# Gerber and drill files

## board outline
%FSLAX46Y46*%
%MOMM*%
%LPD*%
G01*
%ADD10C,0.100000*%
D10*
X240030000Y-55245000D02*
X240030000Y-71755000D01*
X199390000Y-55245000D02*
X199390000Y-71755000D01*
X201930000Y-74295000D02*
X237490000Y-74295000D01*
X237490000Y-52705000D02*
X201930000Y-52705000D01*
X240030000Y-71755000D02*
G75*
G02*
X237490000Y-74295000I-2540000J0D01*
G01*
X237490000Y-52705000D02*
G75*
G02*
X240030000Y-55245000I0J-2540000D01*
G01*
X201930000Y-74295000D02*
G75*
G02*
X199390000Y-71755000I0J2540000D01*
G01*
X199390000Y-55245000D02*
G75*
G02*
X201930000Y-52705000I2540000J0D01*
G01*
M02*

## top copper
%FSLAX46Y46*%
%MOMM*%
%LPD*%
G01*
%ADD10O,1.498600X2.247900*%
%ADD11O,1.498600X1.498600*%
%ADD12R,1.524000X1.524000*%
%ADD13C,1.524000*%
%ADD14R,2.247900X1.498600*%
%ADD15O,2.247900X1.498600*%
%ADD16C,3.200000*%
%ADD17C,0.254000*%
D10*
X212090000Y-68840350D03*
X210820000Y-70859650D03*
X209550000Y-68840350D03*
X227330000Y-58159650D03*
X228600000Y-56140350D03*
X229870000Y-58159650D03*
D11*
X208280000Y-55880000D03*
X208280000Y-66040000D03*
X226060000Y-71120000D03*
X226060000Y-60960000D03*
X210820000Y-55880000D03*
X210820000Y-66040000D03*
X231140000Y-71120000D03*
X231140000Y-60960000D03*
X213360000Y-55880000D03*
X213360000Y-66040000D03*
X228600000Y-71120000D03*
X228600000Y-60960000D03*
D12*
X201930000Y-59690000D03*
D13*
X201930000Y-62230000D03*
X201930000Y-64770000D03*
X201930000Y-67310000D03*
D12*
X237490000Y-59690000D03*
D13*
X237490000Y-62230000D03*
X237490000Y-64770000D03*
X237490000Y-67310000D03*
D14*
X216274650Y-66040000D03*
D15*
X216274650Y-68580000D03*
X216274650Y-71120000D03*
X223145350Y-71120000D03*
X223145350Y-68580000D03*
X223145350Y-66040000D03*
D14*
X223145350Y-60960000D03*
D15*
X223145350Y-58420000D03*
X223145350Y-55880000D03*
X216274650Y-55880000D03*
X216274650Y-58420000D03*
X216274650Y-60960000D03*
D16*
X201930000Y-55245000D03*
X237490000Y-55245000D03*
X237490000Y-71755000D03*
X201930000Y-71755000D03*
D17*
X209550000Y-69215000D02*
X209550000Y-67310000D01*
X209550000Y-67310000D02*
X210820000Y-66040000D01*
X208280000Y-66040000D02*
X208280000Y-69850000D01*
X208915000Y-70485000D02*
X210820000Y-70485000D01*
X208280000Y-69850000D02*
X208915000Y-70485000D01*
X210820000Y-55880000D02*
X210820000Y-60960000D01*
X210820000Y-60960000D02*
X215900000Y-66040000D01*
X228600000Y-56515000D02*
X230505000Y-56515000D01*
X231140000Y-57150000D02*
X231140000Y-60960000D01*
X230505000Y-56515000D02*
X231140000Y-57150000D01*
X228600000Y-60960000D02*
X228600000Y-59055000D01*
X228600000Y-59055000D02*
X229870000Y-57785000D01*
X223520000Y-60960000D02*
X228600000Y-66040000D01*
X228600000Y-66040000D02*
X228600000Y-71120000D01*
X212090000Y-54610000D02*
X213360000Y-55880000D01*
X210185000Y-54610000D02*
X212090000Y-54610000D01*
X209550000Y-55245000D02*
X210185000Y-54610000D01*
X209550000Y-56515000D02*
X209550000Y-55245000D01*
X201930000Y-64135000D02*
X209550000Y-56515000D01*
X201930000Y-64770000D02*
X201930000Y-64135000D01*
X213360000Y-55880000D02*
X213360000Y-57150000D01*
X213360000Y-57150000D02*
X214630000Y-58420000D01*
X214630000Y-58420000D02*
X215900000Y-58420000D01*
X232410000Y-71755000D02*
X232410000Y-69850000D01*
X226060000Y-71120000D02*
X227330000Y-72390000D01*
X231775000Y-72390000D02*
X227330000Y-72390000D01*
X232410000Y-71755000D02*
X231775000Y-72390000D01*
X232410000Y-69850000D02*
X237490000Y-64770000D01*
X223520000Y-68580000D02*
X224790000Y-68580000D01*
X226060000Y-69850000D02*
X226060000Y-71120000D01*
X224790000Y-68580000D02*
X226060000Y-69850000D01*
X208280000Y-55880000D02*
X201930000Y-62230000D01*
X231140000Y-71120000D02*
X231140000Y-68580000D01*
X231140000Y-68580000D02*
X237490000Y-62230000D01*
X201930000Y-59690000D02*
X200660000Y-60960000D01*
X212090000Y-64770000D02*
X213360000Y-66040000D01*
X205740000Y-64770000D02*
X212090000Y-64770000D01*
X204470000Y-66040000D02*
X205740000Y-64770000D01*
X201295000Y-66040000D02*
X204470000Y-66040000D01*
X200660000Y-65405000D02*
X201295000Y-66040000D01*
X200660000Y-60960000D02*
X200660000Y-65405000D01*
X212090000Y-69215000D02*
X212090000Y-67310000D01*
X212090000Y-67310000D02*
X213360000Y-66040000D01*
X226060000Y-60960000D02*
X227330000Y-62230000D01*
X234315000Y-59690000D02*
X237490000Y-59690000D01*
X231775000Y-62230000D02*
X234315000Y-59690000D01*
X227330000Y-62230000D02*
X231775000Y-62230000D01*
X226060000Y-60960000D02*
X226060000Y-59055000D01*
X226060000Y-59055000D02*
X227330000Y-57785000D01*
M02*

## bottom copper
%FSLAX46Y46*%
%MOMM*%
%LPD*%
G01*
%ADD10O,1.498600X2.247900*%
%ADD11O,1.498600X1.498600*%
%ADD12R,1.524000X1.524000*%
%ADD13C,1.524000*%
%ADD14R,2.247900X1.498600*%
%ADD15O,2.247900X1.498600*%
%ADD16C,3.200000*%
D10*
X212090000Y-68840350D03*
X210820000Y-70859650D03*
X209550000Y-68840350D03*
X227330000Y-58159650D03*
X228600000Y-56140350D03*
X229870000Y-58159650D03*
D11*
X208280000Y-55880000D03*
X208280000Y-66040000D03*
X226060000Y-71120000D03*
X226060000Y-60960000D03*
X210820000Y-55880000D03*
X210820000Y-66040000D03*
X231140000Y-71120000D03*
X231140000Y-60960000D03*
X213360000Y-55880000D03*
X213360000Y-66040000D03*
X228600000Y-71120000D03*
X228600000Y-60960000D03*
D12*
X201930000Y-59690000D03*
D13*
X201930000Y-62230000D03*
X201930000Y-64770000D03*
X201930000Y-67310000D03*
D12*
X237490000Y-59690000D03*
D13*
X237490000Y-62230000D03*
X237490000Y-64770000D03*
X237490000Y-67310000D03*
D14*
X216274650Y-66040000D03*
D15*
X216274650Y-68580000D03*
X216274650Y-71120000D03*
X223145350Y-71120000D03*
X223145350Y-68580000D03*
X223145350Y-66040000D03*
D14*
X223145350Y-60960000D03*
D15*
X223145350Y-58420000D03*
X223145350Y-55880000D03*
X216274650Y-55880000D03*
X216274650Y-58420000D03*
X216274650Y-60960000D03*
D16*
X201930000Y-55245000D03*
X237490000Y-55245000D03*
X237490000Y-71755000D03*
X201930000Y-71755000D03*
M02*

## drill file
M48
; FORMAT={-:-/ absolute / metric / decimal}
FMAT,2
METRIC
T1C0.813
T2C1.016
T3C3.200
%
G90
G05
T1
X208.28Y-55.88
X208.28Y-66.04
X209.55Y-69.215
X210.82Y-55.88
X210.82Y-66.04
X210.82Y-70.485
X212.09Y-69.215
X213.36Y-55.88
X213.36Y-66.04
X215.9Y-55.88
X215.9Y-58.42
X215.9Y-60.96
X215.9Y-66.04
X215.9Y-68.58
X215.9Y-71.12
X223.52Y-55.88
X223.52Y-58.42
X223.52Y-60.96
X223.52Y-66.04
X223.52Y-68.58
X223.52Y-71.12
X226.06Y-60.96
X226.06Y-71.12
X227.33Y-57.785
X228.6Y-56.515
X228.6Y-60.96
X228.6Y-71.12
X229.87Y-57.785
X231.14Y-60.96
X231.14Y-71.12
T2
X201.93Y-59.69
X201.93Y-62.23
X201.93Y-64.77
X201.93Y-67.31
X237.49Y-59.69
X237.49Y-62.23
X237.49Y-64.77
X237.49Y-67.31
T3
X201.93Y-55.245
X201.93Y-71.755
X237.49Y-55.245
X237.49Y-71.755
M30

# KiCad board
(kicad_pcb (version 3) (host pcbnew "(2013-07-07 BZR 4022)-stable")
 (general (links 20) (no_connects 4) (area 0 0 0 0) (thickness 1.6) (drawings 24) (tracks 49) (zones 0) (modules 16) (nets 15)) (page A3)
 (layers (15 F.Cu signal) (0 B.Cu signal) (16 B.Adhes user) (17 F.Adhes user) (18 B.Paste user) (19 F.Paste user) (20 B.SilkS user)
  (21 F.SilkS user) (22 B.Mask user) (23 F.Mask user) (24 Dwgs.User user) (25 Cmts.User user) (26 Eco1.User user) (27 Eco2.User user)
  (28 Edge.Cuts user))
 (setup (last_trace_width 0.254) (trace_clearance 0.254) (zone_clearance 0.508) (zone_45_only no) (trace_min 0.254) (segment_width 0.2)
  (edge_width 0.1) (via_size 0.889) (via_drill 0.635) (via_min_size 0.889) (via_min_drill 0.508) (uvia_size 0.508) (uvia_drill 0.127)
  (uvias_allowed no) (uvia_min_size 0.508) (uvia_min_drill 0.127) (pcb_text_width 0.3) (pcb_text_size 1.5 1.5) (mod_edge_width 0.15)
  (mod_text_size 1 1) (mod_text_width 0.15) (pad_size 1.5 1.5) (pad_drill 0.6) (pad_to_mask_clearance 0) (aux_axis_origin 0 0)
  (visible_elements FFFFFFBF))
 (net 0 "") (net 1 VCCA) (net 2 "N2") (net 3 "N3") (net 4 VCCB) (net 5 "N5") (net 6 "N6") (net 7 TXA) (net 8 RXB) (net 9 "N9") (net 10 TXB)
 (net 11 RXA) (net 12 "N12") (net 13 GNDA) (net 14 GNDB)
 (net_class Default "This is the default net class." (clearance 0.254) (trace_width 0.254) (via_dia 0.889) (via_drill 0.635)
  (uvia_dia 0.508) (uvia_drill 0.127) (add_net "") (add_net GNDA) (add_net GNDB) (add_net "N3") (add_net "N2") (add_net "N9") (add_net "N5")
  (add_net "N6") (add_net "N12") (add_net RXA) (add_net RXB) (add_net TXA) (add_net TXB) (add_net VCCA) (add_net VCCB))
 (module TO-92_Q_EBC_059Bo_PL (layer F.Cu) (at 212.09 69.215)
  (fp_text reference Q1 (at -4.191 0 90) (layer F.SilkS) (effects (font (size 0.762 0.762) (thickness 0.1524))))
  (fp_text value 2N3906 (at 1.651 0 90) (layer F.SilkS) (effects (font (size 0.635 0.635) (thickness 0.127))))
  (pad 1 thru_hole oval (at 0 0) (size 1.4986 2.2479) (drill 0.8128 (offset 0 -0.37465)) (layers *.Cu *.Mask F.SilkS) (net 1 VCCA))
  (pad 2 thru_hole oval (at -1.27 1.27) (size 1.4986 2.2479) (drill 0.8128 (offset 0 0.37465)) (layers *.Cu *.Mask F.SilkS) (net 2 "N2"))
  (pad 3 thru_hole oval (at -2.54 0) (size 1.4986 2.2479) (drill 0.8128 (offset 0 -0.37465)) (layers *.Cu *.Mask F.SilkS) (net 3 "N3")))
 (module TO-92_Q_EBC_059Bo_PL (layer F.Cu) (at 227.33 57.785 180)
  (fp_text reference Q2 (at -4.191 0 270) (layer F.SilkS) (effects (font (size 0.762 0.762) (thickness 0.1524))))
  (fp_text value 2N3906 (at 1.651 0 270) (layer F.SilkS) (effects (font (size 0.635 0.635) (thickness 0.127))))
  (pad 1 thru_hole oval (at 0 0 180) (size 1.4986 2.2479) (drill 0.8128 (offset 0 -0.37465)) (layers *.Cu *.Mask F.SilkS) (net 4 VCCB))
  (pad 2 thru_hole oval (at -1.27 1.27 180) (size 1.4986 2.2479) (drill 0.8128 (offset 0 0.37465)) (layers *.Cu *.Mask F.SilkS) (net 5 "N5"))
  (pad 3 thru_hole oval (at -2.54 0 180) (size 1.4986 2.2479) (drill 0.8128 (offset 0 -0.37465)) (layers *.Cu *.Mask F.SilkS) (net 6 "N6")))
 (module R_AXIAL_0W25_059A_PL (layer F.Cu) (at 208.28 55.88 270) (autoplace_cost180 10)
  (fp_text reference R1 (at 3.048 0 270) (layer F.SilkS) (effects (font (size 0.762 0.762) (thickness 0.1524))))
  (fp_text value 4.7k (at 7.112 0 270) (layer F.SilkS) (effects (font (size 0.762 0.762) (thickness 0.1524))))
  (pad 1 thru_hole oval (at 0 0 270) (size 1.4986 1.4986) (drill 0.8128) (layers *.Cu *.Mask F.SilkS) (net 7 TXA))
  (pad 2 thru_hole oval (at 10.16 0 270) (size 1.4986 1.4986) (drill 0.8128) (layers *.Cu *.Mask F.SilkS) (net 2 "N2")))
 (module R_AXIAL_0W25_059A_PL (layer F.Cu) (at 226.06 71.12 90) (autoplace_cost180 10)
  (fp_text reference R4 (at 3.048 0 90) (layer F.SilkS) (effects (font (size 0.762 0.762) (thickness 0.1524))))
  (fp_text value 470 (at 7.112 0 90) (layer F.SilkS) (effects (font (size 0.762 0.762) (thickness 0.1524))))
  (pad 1 thru_hole oval (at 0 0 90) (size 1.4986 1.4986) (drill 0.8128) (layers *.Cu *.Mask F.SilkS) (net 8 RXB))
  (pad 2 thru_hole oval (at 10.16 0 90) (size 1.4986 1.4986) (drill 0.8128) (layers *.Cu *.Mask F.SilkS) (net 4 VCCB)))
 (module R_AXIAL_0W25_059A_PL (layer F.Cu) (at 210.82 55.88 270) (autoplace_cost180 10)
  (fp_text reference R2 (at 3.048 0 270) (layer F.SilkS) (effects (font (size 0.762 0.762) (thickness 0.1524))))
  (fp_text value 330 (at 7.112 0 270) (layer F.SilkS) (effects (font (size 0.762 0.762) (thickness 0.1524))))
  (pad 1 thru_hole oval (at 0 0 270) (size 1.4986 1.4986) (drill 0.8128) (layers *.Cu *.Mask F.SilkS) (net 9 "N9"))
  (pad 2 thru_hole oval (at 10.16 0 270) (size 1.4986 1.4986) (drill 0.8128) (layers *.Cu *.Mask F.SilkS) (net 3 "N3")))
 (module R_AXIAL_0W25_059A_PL (layer F.Cu) (at 231.14 71.12 90) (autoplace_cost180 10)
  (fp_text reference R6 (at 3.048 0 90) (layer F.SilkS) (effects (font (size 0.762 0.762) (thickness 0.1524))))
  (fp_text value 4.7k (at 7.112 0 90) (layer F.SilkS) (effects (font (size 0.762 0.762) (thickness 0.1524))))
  (pad 1 thru_hole oval (at 0 0 90) (size 1.4986 1.4986) (drill 0.8128) (layers *.Cu *.Mask F.SilkS) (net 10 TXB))
  (pad 2 thru_hole oval (at 10.16 0 90) (size 1.4986 1.4986) (drill 0.8128) (layers *.Cu *.Mask F.SilkS) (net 5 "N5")))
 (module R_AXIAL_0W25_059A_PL (layer F.Cu) (at 213.36 55.88 270) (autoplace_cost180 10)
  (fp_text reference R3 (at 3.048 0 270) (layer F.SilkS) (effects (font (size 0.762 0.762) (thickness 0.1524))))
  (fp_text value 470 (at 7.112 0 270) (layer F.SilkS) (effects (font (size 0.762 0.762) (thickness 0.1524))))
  (pad 1 thru_hole oval (at 0 0 270) (size 1.4986 1.4986) (drill 0.8128) (layers *.Cu *.Mask F.SilkS) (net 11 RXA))
  (pad 2 thru_hole oval (at 10.16 0 270) (size 1.4986 1.4986) (drill 0.8128) (layers *.Cu *.Mask F.SilkS) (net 1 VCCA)))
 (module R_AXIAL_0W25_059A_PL (layer F.Cu) (at 228.6 71.12 90) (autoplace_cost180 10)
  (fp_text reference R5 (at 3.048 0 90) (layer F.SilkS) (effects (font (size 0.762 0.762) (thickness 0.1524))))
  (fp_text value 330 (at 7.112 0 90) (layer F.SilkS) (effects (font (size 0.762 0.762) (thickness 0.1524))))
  (pad 1 thru_hole oval (at 0 0 90) (size 1.4986 1.4986) (drill 0.8128) (layers *.Cu *.Mask F.SilkS) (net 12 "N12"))
  (pad 2 thru_hole oval (at 10.16 0 90) (size 1.4986 1.4986) (drill 0.8128) (layers *.Cu *.Mask F.SilkS) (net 6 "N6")))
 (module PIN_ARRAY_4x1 (layer F.Cu) (at 201.93 63.5 270)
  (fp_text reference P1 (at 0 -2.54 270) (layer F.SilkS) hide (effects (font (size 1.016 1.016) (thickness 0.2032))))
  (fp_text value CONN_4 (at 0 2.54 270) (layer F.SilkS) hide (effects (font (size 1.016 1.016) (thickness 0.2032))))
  (pad 1 thru_hole rect (at -3.81 0 270) (size 1.524 1.524) (drill 1.016) (layers *.Cu *.Mask F.SilkS) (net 1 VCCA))
  (pad 2 thru_hole circle (at -1.27 0 270) (size 1.524 1.524) (drill 1.016) (layers *.Cu *.Mask F.SilkS) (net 7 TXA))
  (pad 3 thru_hole circle (at 1.27 0 270) (size 1.524 1.524) (drill 1.016) (layers *.Cu *.Mask F.SilkS) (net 11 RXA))
  (pad 4 thru_hole circle (at 3.81 0 270) (size 1.524 1.524) (drill 1.016) (layers *.Cu *.Mask F.SilkS) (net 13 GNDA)))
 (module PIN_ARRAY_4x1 (layer F.Cu) (at 237.49 63.5 270)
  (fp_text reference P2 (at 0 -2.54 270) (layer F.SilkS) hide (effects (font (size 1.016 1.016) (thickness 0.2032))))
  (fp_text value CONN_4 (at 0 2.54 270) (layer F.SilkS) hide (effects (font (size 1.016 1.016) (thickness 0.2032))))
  (pad 1 thru_hole rect (at -3.81 0 270) (size 1.524 1.524) (drill 1.016) (layers *.Cu *.Mask F.SilkS) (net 4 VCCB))
  (pad 2 thru_hole circle (at -1.27 0 270) (size 1.524 1.524) (drill 1.016) (layers *.Cu *.Mask F.SilkS) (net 10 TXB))
  (pad 3 thru_hole circle (at 1.27 0 270) (size 1.524 1.524) (drill 1.016) (layers *.Cu *.Mask F.SilkS) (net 8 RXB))
  (pad 4 thru_hole circle (at 3.81 0 270) (size 1.524 1.524) (drill 1.016) (layers *.Cu *.Mask F.SilkS) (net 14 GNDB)))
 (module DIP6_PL (layer F.Cu) (at 215.9 66.04 270)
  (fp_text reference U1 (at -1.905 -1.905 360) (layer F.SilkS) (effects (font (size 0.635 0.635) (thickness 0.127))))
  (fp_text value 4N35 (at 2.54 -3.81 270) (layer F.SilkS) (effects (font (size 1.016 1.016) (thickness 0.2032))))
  (pad 1 thru_hole rect (at 0 0 270) (size 1.4986 2.2479) (drill 0.8128 (offset 0 -0.37465)) (layers *.Cu *.Mask F.SilkS) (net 9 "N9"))
  (pad 2 thru_hole oval (at 2.54 0 270) (size 1.4986 2.2479) (drill 0.8128 (offset 0 -0.37465)) (layers *.Cu *.Mask F.SilkS) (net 13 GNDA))
  (pad 3 thru_hole oval (at 5.08 0 270) (size 1.4986 2.2479) (drill 0.8128 (offset 0 -0.37465)) (layers *.Cu *.Mask F.SilkS))
  (pad 4 thru_hole oval (at 5.08 -7.62 270) (size 1.4986 2.2479) (drill 0.8128 (offset 0 0.37465)) (layers *.Cu *.Mask F.SilkS)
   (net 14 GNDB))
  (pad 5 thru_hole oval (at 2.54 -7.62 270) (size 1.4986 2.2479) (drill 0.8128 (offset 0 0.37465)) (layers *.Cu *.Mask F.SilkS) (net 8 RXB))
  (pad 6 thru_hole oval (at 0 -7.62 270) (size 1.4986 2.2479) (drill 0.8128 (offset 0 0.37465)) (layers *.Cu *.Mask F.SilkS)))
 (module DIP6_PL (layer F.Cu) (at 223.52 60.96 90)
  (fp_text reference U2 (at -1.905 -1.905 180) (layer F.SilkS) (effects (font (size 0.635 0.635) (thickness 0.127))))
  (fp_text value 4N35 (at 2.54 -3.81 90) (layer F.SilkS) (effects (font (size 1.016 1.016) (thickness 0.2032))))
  (pad 1 thru_hole rect (at 0 0 90) (size 1.4986 2.2479) (drill 0.8128 (offset 0 -0.37465)) (layers *.Cu *.Mask F.SilkS) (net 12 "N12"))
  (pad 2 thru_hole oval (at 2.54 0 90) (size 1.4986 2.2479) (drill 0.8128 (offset 0 -0.37465)) (layers *.Cu *.Mask F.SilkS) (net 14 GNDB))
  (pad 3 thru_hole oval (at 5.08 0 90) (size 1.4986 2.2479) (drill 0.8128 (offset 0 -0.37465)) (layers *.Cu *.Mask F.SilkS))
  (pad 4 thru_hole oval (at 5.08 -7.62 90) (size 1.4986 2.2479) (drill 0.8128 (offset 0 0.37465)) (layers *.Cu *.Mask F.SilkS) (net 13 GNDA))
  (pad 5 thru_hole oval (at 2.54 -7.62 90) (size 1.4986 2.2479) (drill 0.8128 (offset 0 0.37465)) (layers *.Cu *.Mask F.SilkS) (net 11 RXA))
  (pad 6 thru_hole oval (at 0 -7.62 90) (size 1.4986 2.2479) (drill 0.8128 (offset 0 0.37465)) (layers *.Cu *.Mask F.SilkS)))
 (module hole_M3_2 (layer F.Cu) (at 201.93 55.245)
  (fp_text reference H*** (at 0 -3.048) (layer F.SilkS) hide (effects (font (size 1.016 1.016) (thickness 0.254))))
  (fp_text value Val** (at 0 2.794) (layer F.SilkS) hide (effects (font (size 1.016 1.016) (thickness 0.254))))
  (pad 1 thru_hole circle (at 0 0) (size 3.2 3.2) (drill 3.2) (layers *.Cu *.Mask F.SilkS)))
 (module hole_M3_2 (layer F.Cu) (at 237.49 55.245)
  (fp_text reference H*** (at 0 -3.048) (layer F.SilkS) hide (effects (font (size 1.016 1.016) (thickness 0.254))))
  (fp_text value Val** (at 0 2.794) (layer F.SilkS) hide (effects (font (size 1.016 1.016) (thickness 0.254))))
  (pad 1 thru_hole circle (at 0 0) (size 3.2 3.2) (drill 3.2) (layers *.Cu *.Mask F.SilkS)))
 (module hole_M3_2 (layer F.Cu) (at 237.49 71.755)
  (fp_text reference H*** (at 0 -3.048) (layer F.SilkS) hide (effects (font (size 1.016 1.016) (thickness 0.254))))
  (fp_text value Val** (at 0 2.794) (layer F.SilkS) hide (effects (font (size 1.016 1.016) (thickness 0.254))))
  (pad 1 thru_hole circle (at 0 0) (size 3.2 3.2) (drill 3.2) (layers *.Cu *.Mask F.SilkS)))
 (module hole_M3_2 (layer F.Cu) (at 201.93 71.755)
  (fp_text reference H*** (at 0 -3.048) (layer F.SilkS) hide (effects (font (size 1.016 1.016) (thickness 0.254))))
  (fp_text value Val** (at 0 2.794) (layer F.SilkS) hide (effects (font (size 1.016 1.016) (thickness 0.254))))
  (pad 1 thru_hole circle (at 0 0) (size 3.2 3.2) (drill 3.2) (layers *.Cu *.Mask F.SilkS)))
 (gr_line (start 240.03 55.245) (end 240.03 71.755) (angle 90) (layer Edge.Cuts) (width 0.1))
 (gr_line (start 199.39 55.245) (end 199.39 71.755) (angle 90) (layer Edge.Cuts) (width 0.1))
 (gr_line (start 201.93 74.295) (end 237.49 74.295) (angle 90) (layer Edge.Cuts) (width 0.1))
 (gr_line (start 237.49 52.705) (end 201.93 52.705) (angle 90) (layer Edge.Cuts) (width 0.1))
 (gr_arc (start 237.49 71.755) (end 240.03 71.755) (angle 90) (layer Edge.Cuts) (width 0.1))
 (gr_arc (start 237.49 55.245) (end 237.49 52.705) (angle 90) (layer Edge.Cuts) (width 0.1))
 (gr_arc (start 201.93 71.755) (end 201.93 74.295) (angle 90) (layer Edge.Cuts) (width 0.1))
 (gr_arc (start 201.93 55.245) (end 199.39 55.245) (angle 90) (layer Edge.Cuts) (width 0.1))
 (segment (start 209.55 69.215) (end 209.55 67.31) (width 0.254) (layer F.Cu) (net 3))
 (segment (start 209.55 67.31) (end 210.82 66.04) (width 0.254) (layer F.Cu) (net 3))
 (segment (start 208.28 66.04) (end 208.28 69.85) (width 0.254) (layer F.Cu) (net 2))
 (segment (start 208.915 70.485) (end 210.82 70.485) (width 0.254) (layer F.Cu) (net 2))
 (segment (start 208.28 69.85) (end 208.915 70.485) (width 0.254) (layer F.Cu) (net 2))
 (segment (start 210.82 55.88) (end 210.82 60.96) (width 0.254) (layer F.Cu) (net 9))
 (segment (start 210.82 60.96) (end 215.9 66.04) (width 0.254) (layer F.Cu) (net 9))
 (segment (start 228.6 56.515) (end 230.505 56.515) (width 0.254) (layer F.Cu) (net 5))
 (segment (start 231.14 57.15) (end 231.14 60.96) (width 0.254) (layer F.Cu) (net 5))
 (segment (start 230.505 56.515) (end 231.14 57.15) (width 0.254) (layer F.Cu) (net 5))
 (segment (start 228.6 60.96) (end 228.6 59.055) (width 0.254) (layer F.Cu) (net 6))
 (segment (start 228.6 59.055) (end 229.87 57.785) (width 0.254) (layer F.Cu) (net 6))
 (segment (start 223.52 60.96) (end 228.6 66.04) (width 0.254) (layer F.Cu) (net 12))
 (segment (start 228.6 66.04) (end 228.6 71.12) (width 0.254) (layer F.Cu) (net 12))
 (segment (start 212.09 54.61) (end 213.36 55.88) (width 0.254) (layer F.Cu) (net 11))
 (segment (start 210.185 54.61) (end 212.09 54.61) (width 0.254) (layer F.Cu) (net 11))
 (segment (start 209.55 55.245) (end 210.185 54.61) (width 0.254) (layer F.Cu) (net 11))
 (segment (start 209.55 56.515) (end 209.55 55.245) (width 0.254) (layer F.Cu) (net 11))
 (segment (start 201.93 64.135) (end 209.55 56.515) (width 0.254) (layer F.Cu) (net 11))
 (segment (start 201.93 64.77) (end 201.93 64.135) (width 0.254) (layer F.Cu) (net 11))
 (segment (start 213.36 55.88) (end 213.36 57.15) (width 0.254) (layer F.Cu) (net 11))
 (segment (start 213.36 57.15) (end 214.63 58.42) (width 0.254) (layer F.Cu) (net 11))
 (segment (start 214.63 58.42) (end 215.9 58.42) (width 0.254) (layer F.Cu) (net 11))
 (segment (start 232.41 71.755) (end 232.41 69.85) (width 0.254) (layer F.Cu) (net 8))
 (segment (start 226.06 71.12) (end 227.33 72.39) (width 0.254) (layer F.Cu) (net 8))
 (segment (start 231.775 72.39) (end 227.33 72.39) (width 0.254) (layer F.Cu) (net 8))
 (segment (start 232.41 71.755) (end 231.775 72.39) (width 0.254) (layer F.Cu) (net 8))
 (segment (start 232.41 69.85) (end 237.49 64.77) (width 0.254) (layer F.Cu) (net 8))
 (segment (start 223.52 68.58) (end 224.79 68.58) (width 0.254) (layer F.Cu) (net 8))
 (segment (start 226.06 69.85) (end 226.06 71.12) (width 0.254) (layer F.Cu) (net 8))
 (segment (start 224.79 68.58) (end 226.06 69.85) (width 0.254) (layer F.Cu) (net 8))
 (segment (start 208.28 55.88) (end 201.93 62.23) (width 0.254) (layer F.Cu) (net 7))
 (segment (start 231.14 71.12) (end 231.14 68.58) (width 0.254) (layer F.Cu) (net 10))
 (segment (start 231.14 68.58) (end 237.49 62.23) (width 0.254) (layer F.Cu) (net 10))
 (segment (start 201.93 59.69) (end 200.66 60.96) (width 0.254) (layer F.Cu) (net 1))
 (segment (start 212.09 64.77) (end 213.36 66.04) (width 0.254) (layer F.Cu) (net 1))
 (segment (start 205.74 64.77) (end 212.09 64.77) (width 0.254) (layer F.Cu) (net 1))
 (segment (start 204.47 66.04) (end 205.74 64.77) (width 0.254) (layer F.Cu) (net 1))
 (segment (start 201.295 66.04) (end 204.47 66.04) (width 0.254) (layer F.Cu) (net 1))
 (segment (start 200.66 65.405) (end 201.295 66.04) (width 0.254) (layer F.Cu) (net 1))
 (segment (start 200.66 60.96) (end 200.66 65.405) (width 0.254) (layer F.Cu) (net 1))
 (segment (start 212.09 69.215) (end 212.09 67.31) (width 0.254) (layer F.Cu) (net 1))
 (segment (start 212.09 67.31) (end 213.36 66.04) (width 0.254) (layer F.Cu) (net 1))
 (segment (start 226.06 60.96) (end 227.33 62.23) (width 0.254) (layer F.Cu) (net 4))
 (segment (start 234.315 59.69) (end 237.49 59.69) (width 0.254) (layer F.Cu) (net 4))
 (segment (start 231.775 62.23) (end 234.315 59.69) (width 0.254) (layer F.Cu) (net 4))
 (segment (start 227.33 62.23) (end 231.775 62.23) (width 0.254) (layer F.Cu) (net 4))
 (segment (start 226.06 60.96) (end 226.06 59.055) (width 0.254) (layer F.Cu) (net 4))
 (segment (start 226.06 59.055) (end 227.33 57.785) (width 0.254) (layer F.Cu) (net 4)))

